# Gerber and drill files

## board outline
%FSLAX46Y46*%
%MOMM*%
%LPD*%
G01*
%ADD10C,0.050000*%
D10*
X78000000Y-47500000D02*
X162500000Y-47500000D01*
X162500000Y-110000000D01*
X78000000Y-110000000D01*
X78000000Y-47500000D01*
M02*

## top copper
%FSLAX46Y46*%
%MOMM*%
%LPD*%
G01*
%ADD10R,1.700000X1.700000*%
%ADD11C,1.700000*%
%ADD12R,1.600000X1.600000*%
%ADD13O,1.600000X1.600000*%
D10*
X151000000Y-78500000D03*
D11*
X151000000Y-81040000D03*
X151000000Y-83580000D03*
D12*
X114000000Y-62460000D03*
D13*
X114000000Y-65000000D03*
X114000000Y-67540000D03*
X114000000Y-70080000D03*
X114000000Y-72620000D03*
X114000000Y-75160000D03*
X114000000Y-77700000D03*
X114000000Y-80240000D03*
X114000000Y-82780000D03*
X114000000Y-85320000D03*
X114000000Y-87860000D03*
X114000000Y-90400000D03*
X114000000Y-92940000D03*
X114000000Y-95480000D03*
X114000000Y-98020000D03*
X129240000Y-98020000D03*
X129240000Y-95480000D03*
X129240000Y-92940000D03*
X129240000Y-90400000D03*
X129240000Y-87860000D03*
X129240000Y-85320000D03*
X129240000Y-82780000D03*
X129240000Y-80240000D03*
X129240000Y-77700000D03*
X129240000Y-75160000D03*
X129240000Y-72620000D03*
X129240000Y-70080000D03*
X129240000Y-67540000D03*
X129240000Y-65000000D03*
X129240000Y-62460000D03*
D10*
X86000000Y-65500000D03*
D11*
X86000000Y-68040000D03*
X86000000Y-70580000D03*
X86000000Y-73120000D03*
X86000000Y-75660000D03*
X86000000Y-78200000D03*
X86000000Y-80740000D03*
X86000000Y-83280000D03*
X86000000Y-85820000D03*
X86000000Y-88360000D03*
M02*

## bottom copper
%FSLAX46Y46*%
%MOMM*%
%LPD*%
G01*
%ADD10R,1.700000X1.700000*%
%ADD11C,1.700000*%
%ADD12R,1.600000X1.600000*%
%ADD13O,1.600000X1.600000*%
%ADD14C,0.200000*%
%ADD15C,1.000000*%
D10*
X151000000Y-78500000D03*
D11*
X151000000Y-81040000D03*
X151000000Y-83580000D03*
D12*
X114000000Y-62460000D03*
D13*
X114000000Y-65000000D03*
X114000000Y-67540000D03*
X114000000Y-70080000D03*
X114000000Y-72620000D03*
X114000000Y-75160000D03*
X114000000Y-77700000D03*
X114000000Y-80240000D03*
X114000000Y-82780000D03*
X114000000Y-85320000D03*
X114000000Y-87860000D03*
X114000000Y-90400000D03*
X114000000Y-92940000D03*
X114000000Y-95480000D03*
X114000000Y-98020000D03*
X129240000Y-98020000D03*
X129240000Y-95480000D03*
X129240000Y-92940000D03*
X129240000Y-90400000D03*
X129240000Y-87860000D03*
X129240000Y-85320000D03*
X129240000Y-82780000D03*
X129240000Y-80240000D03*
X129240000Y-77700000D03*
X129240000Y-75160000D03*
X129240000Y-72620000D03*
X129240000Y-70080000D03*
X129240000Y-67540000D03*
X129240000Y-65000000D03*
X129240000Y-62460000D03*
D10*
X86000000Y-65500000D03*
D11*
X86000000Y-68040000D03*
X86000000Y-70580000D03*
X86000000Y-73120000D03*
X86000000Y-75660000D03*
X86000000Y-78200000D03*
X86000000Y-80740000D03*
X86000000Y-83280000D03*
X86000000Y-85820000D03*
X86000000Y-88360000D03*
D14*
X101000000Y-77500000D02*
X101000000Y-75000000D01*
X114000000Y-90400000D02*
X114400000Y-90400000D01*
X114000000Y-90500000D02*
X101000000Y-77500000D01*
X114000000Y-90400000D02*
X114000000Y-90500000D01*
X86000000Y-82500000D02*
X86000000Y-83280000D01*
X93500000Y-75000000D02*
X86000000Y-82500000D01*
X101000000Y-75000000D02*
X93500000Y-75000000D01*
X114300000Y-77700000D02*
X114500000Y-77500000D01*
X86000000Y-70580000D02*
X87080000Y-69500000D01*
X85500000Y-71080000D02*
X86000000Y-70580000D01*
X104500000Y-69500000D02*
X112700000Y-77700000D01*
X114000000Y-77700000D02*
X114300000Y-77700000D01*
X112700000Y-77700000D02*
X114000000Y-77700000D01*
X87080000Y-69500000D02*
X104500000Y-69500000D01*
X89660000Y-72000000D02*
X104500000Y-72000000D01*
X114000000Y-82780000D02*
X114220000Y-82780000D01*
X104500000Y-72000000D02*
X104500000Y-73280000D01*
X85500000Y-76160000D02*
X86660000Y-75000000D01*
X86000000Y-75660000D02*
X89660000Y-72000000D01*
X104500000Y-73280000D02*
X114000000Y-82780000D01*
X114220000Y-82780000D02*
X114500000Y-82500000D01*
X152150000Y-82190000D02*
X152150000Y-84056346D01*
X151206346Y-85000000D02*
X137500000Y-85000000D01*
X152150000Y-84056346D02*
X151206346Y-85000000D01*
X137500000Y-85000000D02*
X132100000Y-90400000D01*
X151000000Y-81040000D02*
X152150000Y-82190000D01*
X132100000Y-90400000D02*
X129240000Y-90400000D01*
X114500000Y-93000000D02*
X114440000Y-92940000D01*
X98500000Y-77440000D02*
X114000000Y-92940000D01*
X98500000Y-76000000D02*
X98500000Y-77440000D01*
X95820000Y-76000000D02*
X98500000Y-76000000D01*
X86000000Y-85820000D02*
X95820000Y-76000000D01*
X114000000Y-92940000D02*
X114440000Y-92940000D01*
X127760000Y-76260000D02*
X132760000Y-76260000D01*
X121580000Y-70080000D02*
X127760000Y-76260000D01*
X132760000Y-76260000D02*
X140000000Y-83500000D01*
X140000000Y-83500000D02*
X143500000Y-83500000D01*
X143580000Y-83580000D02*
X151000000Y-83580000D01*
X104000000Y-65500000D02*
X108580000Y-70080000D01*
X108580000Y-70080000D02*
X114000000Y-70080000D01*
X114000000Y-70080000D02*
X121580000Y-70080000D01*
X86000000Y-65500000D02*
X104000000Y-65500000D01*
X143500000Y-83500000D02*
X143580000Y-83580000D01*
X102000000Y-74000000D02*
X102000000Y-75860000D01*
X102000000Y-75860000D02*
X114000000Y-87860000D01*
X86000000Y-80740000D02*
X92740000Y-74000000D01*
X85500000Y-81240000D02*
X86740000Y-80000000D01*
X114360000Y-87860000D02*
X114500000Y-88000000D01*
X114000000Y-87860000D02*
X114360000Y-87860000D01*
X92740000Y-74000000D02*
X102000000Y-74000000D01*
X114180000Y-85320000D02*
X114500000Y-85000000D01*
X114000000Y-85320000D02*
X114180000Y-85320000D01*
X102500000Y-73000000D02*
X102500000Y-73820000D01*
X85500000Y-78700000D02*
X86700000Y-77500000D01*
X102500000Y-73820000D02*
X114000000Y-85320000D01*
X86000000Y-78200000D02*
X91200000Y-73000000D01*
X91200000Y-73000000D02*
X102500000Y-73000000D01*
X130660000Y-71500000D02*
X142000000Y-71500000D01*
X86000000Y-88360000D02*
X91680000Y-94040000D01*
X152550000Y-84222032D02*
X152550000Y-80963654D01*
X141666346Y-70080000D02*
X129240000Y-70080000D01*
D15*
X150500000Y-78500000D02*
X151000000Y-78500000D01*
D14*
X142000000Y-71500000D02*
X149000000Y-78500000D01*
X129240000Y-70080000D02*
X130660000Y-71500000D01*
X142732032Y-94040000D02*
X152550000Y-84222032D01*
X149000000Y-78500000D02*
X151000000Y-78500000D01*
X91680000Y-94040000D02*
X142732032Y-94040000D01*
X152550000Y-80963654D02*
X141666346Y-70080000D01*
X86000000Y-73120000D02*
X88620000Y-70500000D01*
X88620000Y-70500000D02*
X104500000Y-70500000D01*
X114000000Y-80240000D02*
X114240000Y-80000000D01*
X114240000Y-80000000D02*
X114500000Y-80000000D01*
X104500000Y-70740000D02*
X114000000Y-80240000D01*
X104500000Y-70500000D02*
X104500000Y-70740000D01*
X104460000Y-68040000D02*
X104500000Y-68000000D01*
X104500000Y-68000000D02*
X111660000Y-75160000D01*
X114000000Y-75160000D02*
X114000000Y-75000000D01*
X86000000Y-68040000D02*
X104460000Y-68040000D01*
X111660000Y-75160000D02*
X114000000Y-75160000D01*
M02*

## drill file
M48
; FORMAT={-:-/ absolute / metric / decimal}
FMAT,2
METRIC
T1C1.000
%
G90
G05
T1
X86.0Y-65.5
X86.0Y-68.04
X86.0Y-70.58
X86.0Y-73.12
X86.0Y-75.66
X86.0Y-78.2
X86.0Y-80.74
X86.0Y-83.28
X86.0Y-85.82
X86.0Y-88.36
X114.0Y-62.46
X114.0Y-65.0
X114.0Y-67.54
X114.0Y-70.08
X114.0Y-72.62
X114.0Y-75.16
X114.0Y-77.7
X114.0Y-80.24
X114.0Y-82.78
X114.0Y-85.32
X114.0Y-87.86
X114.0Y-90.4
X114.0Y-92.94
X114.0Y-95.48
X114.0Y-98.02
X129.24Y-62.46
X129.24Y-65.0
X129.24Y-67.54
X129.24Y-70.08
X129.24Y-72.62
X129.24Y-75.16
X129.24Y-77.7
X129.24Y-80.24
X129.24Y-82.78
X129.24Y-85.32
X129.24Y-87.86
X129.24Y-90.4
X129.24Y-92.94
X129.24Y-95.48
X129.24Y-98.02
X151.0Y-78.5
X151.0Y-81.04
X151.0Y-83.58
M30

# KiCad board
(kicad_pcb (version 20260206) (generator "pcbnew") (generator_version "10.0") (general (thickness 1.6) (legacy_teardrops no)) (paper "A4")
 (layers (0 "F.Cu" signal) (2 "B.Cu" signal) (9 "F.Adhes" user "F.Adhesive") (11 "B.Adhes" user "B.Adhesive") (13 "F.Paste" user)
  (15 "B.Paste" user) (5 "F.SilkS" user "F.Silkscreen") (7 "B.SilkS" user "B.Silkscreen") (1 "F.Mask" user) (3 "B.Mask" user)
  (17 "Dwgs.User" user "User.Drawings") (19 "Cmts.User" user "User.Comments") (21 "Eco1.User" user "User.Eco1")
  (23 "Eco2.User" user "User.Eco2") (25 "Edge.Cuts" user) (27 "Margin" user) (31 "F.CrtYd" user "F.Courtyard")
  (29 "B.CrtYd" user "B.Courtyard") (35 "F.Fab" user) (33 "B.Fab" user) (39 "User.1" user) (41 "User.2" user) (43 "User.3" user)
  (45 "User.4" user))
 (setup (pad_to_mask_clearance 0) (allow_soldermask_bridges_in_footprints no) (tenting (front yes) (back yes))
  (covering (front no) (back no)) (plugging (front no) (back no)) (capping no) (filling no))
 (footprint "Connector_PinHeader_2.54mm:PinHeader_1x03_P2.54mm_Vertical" (layer "F.Cu") (at 151 78.5)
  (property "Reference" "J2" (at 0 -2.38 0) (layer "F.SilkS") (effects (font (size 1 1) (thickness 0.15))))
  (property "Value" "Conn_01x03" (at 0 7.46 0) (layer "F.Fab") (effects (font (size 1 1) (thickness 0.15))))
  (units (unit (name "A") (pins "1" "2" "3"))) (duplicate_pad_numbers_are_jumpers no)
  (pad "1" thru_hole rect (at 0 0) (size 1.7 1.7) (drill 1) (layers "*.Cu" "*.Mask") (remove_unused_layers no) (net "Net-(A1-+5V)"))
  (pad "2" thru_hole circle (at 0 2.54) (size 1.7 1.7) (drill 1) (layers "*.Cu" "*.Mask") (remove_unused_layers no) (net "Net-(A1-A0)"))
  (pad "3" thru_hole circle (at 0 5.08) (size 1.7 1.7) (drill 1) (layers "*.Cu" "*.Mask") (remove_unused_layers no) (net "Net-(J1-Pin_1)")))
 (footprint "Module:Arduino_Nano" (layer "F.Cu") (at 114 62.46)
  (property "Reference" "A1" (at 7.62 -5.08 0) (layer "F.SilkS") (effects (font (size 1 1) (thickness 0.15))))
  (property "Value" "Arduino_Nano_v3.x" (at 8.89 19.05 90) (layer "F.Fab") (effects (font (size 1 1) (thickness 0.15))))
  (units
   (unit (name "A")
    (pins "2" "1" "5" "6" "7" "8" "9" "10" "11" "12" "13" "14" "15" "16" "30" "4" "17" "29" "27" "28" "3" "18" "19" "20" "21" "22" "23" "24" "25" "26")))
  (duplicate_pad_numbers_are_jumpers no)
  (pad "1" thru_hole rect (at 0 0) (size 1.6 1.6) (drill 1) (layers "*.Cu" "*.Mask") (remove_unused_layers no)
   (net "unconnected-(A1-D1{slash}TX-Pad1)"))
  (pad "2" thru_hole oval (at 0 2.54) (size 1.6 1.6) (drill 1) (layers "*.Cu" "*.Mask") (remove_unused_layers no)
   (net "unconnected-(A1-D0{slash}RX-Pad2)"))
  (pad "3" thru_hole oval (at 0 5.08) (size 1.6 1.6) (drill 1) (layers "*.Cu" "*.Mask") (remove_unused_layers no)
   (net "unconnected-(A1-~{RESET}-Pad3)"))
  (pad "4" thru_hole oval (at 0 7.62) (size 1.6 1.6) (drill 1) (layers "*.Cu" "*.Mask") (remove_unused_layers no) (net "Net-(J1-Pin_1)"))
  (pad "5" thru_hole oval (at 0 10.16) (size 1.6 1.6) (drill 1) (layers "*.Cu" "*.Mask") (remove_unused_layers no)
   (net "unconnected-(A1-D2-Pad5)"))
  (pad "6" thru_hole oval (at 0 12.7) (size 1.6 1.6) (drill 1) (layers "*.Cu" "*.Mask") (remove_unused_layers no) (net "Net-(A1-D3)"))
  (pad "7" thru_hole oval (at 0 15.24) (size 1.6 1.6) (drill 1) (layers "*.Cu" "*.Mask") (remove_unused_layers no) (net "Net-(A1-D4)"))
  (pad "8" thru_hole oval (at 0 17.78) (size 1.6 1.6) (drill 1) (layers "*.Cu" "*.Mask") (remove_unused_layers no) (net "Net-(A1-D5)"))
  (pad "9" thru_hole oval (at 0 20.32) (size 1.6 1.6) (drill 1) (layers "*.Cu" "*.Mask") (remove_unused_layers no) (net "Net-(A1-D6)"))
  (pad "10" thru_hole oval (at 0 22.86) (size 1.6 1.6) (drill 1) (layers "*.Cu" "*.Mask") (remove_unused_layers no) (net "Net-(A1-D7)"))
  (pad "11" thru_hole oval (at 0 25.4) (size 1.6 1.6) (drill 1) (layers "*.Cu" "*.Mask") (remove_unused_layers no) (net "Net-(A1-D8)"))
  (pad "12" thru_hole oval (at 0 27.94) (size 1.6 1.6) (drill 1) (layers "*.Cu" "*.Mask") (remove_unused_layers no) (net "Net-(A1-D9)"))
  (pad "13" thru_hole oval (at 0 30.48) (size 1.6 1.6) (drill 1) (layers "*.Cu" "*.Mask") (remove_unused_layers no) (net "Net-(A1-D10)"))
  (pad "14" thru_hole oval (at 0 33.02) (size 1.6 1.6) (drill 1) (layers "*.Cu" "*.Mask") (remove_unused_layers no)
   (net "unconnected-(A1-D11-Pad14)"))
  (pad "15" thru_hole oval (at 0 35.56) (size 1.6 1.6) (drill 1) (layers "*.Cu" "*.Mask") (remove_unused_layers no)
   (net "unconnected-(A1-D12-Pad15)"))
  (pad "16" thru_hole oval (at 15.24 35.56) (size 1.6 1.6) (drill 1) (layers "*.Cu" "*.Mask") (remove_unused_layers no)
   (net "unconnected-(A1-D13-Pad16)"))
  (pad "17" thru_hole oval (at 15.24 33.02) (size 1.6 1.6) (drill 1) (layers "*.Cu" "*.Mask") (remove_unused_layers no)
   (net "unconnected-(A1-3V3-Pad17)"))
  (pad "18" thru_hole oval (at 15.24 30.48) (size 1.6 1.6) (drill 1) (layers "*.Cu" "*.Mask") (remove_unused_layers no)
   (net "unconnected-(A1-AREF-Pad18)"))
  (pad "19" thru_hole oval (at 15.24 27.94) (size 1.6 1.6) (drill 1) (layers "*.Cu" "*.Mask") (remove_unused_layers no) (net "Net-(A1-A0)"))
  (pad "20" thru_hole oval (at 15.24 25.4) (size 1.6 1.6) (drill 1) (layers "*.Cu" "*.Mask") (remove_unused_layers no)
   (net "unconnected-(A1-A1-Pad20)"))
  (pad "21" thru_hole oval (at 15.24 22.86) (size 1.6 1.6) (drill 1) (layers "*.Cu" "*.Mask") (remove_unused_layers no)
   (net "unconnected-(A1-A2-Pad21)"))
  (pad "22" thru_hole oval (at 15.24 20.32) (size 1.6 1.6) (drill 1) (layers "*.Cu" "*.Mask") (remove_unused_layers no)
   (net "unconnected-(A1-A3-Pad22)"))
  (pad "23" thru_hole oval (at 15.24 17.78) (size 1.6 1.6) (drill 1) (layers "*.Cu" "*.Mask") (remove_unused_layers no)
   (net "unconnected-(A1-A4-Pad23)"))
  (pad "24" thru_hole oval (at 15.24 15.24) (size 1.6 1.6) (drill 1) (layers "*.Cu" "*.Mask") (remove_unused_layers no)
   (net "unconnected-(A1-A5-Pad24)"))
  (pad "25" thru_hole oval (at 15.24 12.7) (size 1.6 1.6) (drill 1) (layers "*.Cu" "*.Mask") (remove_unused_layers no)
   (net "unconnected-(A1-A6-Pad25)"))
  (pad "26" thru_hole oval (at 15.24 10.16) (size 1.6 1.6) (drill 1) (layers "*.Cu" "*.Mask") (remove_unused_layers no)
   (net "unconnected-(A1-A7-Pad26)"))
  (pad "27" thru_hole oval (at 15.24 7.62) (size 1.6 1.6) (drill 1) (layers "*.Cu" "*.Mask") (remove_unused_layers no) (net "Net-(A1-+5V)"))
  (pad "28" thru_hole oval (at 15.24 5.08) (size 1.6 1.6) (drill 1) (layers "*.Cu" "*.Mask") (remove_unused_layers no)
   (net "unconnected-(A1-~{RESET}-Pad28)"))
  (pad "29" thru_hole oval (at 15.24 2.54) (size 1.6 1.6) (drill 1) (layers "*.Cu" "*.Mask") (remove_unused_layers no)
   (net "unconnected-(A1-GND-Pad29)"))
  (pad "30" thru_hole oval (at 15.24 0) (size 1.6 1.6) (drill 1) (layers "*.Cu" "*.Mask") (remove_unused_layers no)
   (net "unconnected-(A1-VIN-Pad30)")))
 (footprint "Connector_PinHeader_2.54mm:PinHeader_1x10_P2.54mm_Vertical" (layer "F.Cu") (at 86 65.5)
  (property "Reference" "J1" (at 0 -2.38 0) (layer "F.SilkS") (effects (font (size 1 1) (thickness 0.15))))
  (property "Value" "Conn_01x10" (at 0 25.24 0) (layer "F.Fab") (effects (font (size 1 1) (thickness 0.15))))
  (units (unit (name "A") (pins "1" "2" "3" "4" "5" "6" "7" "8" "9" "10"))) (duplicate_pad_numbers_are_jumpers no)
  (pad "1" thru_hole rect (at 0 0) (size 1.7 1.7) (drill 1) (layers "*.Cu" "*.Mask") (remove_unused_layers no) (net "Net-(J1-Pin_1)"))
  (pad "2" thru_hole circle (at 0 2.54) (size 1.7 1.7) (drill 1) (layers "*.Cu" "*.Mask") (remove_unused_layers no) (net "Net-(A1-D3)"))
  (pad "3" thru_hole circle (at 0 5.08) (size 1.7 1.7) (drill 1) (layers "*.Cu" "*.Mask") (remove_unused_layers no) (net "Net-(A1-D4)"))
  (pad "4" thru_hole circle (at 0 7.62) (size 1.7 1.7) (drill 1) (layers "*.Cu" "*.Mask") (remove_unused_layers no) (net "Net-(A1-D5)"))
  (pad "5" thru_hole circle (at 0 10.16) (size 1.7 1.7) (drill 1) (layers "*.Cu" "*.Mask") (remove_unused_layers no) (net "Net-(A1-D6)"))
  (pad "6" thru_hole circle (at 0 12.7) (size 1.7 1.7) (drill 1) (layers "*.Cu" "*.Mask") (remove_unused_layers no) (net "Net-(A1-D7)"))
  (pad "7" thru_hole circle (at 0 15.24) (size 1.7 1.7) (drill 1) (layers "*.Cu" "*.Mask") (remove_unused_layers no) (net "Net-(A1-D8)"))
  (pad "8" thru_hole circle (at 0 17.78) (size 1.7 1.7) (drill 1) (layers "*.Cu" "*.Mask") (remove_unused_layers no) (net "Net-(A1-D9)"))
  (pad "9" thru_hole circle (at 0 20.32) (size 1.7 1.7) (drill 1) (layers "*.Cu" "*.Mask") (remove_unused_layers no) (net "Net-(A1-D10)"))
  (pad "10" thru_hole circle (at 0 22.86) (size 1.7 1.7) (drill 1) (layers "*.Cu" "*.Mask") (remove_unused_layers no) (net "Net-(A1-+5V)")))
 (gr_rect (start 78 47.5) (end 162.5 110) (stroke (width 0.05) (type default)) (fill no) (layer "Edge.Cuts"))
 (segment (start 101 77.5) (end 101 75) (width 0.2) (layer "B.Cu") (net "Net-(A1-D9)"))
 (segment (start 114 90.4) (end 114.4 90.4) (width 0.2) (layer "B.Cu") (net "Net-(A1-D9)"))
 (segment (start 114 90.5) (end 101 77.5) (width 0.2) (layer "B.Cu") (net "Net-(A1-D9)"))
 (segment (start 114 90.4) (end 114 90.5) (width 0.2) (layer "B.Cu") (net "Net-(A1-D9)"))
 (segment (start 86 82.5) (end 86 83.28) (width 0.2) (layer "B.Cu") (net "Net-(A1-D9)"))
 (segment (start 93.5 75) (end 86 82.5) (width 0.2) (layer "B.Cu") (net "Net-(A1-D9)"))
 (segment (start 101 75) (end 93.5 75) (width 0.2) (layer "B.Cu") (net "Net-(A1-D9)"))
 (segment (start 114.3 77.7) (end 114.5 77.5) (width 0.2) (layer "B.Cu") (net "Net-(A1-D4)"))
 (segment (start 86 70.58) (end 87.08 69.5) (width 0.2) (layer "B.Cu") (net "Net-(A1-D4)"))
 (segment (start 85.5 71.08) (end 86 70.58) (width 0.2) (layer "B.Cu") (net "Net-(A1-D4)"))
 (segment (start 104.5 69.5) (end 112.7 77.7) (width 0.2) (layer "B.Cu") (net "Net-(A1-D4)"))
 (segment (start 114 77.7) (end 114.3 77.7) (width 0.2) (layer "B.Cu") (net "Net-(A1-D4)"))
 (segment (start 112.7 77.7) (end 114 77.7) (width 0.2) (layer "B.Cu") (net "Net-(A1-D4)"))
 (segment (start 87.08 69.5) (end 104.5 69.5) (width 0.2) (layer "B.Cu") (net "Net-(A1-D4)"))
 (segment (start 89.66 72) (end 104.5 72) (width 0.2) (layer "B.Cu") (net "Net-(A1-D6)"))
 (segment (start 114 82.78) (end 114.22 82.78) (width 0.2) (layer "B.Cu") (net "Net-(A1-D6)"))
 (segment (start 104.5 72) (end 104.5 73.28) (width 0.2) (layer "B.Cu") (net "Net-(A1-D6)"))
 (segment (start 85.5 76.16) (end 86.66 75) (width 0.2) (layer "B.Cu") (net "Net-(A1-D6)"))
 (segment (start 86 75.66) (end 89.66 72) (width 0.2) (layer "B.Cu") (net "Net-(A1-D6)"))
 (segment (start 104.5 73.28) (end 114 82.78) (width 0.2) (layer "B.Cu") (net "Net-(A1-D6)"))
 (segment (start 114.22 82.78) (end 114.5 82.5) (width 0.2) (layer "B.Cu") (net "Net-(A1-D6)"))
 (segment (start 152.15 82.19) (end 152.15 84.056346) (width 0.2) (layer "B.Cu") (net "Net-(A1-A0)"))
 (segment (start 151.206346 85) (end 137.5 85) (width 0.2) (layer "B.Cu") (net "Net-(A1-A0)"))
 (segment (start 152.15 84.056346) (end 151.206346 85) (width 0.2) (layer "B.Cu") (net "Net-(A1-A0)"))
 (segment (start 137.5 85) (end 132.1 90.4) (width 0.2) (layer "B.Cu") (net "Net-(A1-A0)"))
 (segment (start 151 81.04) (end 152.15 82.19) (width 0.2) (layer "B.Cu") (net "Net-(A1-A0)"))
 (segment (start 132.1 90.4) (end 129.24 90.4) (width 0.2) (layer "B.Cu") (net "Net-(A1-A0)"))
 (segment (start 114.5 93) (end 114.44 92.94) (width 0.2) (layer "B.Cu") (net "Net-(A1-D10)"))
 (segment (start 98.5 77.44) (end 114 92.94) (width 0.2) (layer "B.Cu") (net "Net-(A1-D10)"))
 (segment (start 98.5 76) (end 98.5 77.44) (width 0.2) (layer "B.Cu") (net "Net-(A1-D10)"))
 (segment (start 95.82 76) (end 98.5 76) (width 0.2) (layer "B.Cu") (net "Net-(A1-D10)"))
 (segment (start 86 85.82) (end 95.82 76) (width 0.2) (layer "B.Cu") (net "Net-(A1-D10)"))
 (segment (start 114 92.94) (end 114.44 92.94) (width 0.2) (layer "B.Cu") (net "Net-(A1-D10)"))
 (segment (start 127.76 76.26) (end 132.76 76.26) (width 0.2) (layer "B.Cu") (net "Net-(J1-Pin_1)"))
 (segment (start 121.58 70.08) (end 127.76 76.26) (width 0.2) (layer "B.Cu") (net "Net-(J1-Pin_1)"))
 (segment (start 132.76 76.26) (end 140 83.5) (width 0.2) (layer "B.Cu") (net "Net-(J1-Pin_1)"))
 (segment (start 140 83.5) (end 143.5 83.5) (width 0.2) (layer "B.Cu") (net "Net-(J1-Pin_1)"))
 (segment (start 143.58 83.58) (end 151 83.58) (width 0.2) (layer "B.Cu") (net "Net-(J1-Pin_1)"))
 (segment (start 104 65.5) (end 108.58 70.08) (width 0.2) (layer "B.Cu") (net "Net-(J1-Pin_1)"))
 (segment (start 108.58 70.08) (end 114 70.08) (width 0.2) (layer "B.Cu") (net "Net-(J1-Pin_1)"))
 (segment (start 114 70.08) (end 121.58 70.08) (width 0.2) (layer "B.Cu") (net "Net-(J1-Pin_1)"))
 (segment (start 86 65.5) (end 104 65.5) (width 0.2) (layer "B.Cu") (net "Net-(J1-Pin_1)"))
 (segment (start 143.5 83.5) (end 143.58 83.58) (width 0.2) (layer "B.Cu") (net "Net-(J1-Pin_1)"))
 (segment (start 102 74) (end 102 75.86) (width 0.2) (layer "B.Cu") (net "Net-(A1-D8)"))
 (segment (start 102 75.86) (end 114 87.86) (width 0.2) (layer "B.Cu") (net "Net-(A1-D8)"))
 (segment (start 86 80.74) (end 92.74 74) (width 0.2) (layer "B.Cu") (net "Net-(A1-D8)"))
 (segment (start 85.5 81.24) (end 86.74 80) (width 0.2) (layer "B.Cu") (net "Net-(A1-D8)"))
 (segment (start 114.36 87.86) (end 114.5 88) (width 0.2) (layer "B.Cu") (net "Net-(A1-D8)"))
 (segment (start 114 87.86) (end 114.36 87.86) (width 0.2) (layer "B.Cu") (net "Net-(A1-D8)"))
 (segment (start 92.74 74) (end 102 74) (width 0.2) (layer "B.Cu") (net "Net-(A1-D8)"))
 (segment (start 114.18 85.32) (end 114.5 85) (width 0.2) (layer "B.Cu") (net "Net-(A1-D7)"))
 (segment (start 114 85.32) (end 114.18 85.32) (width 0.2) (layer "B.Cu") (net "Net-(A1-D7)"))
 (segment (start 102.5 73) (end 102.5 73.82) (width 0.2) (layer "B.Cu") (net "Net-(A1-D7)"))
 (segment (start 85.5 78.7) (end 86.7 77.5) (width 0.2) (layer "B.Cu") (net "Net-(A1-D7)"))
 (segment (start 102.5 73.82) (end 114 85.32) (width 0.2) (layer "B.Cu") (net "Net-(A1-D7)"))
 (segment (start 86 78.2) (end 91.2 73) (width 0.2) (layer "B.Cu") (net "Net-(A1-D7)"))
 (segment (start 91.2 73) (end 102.5 73) (width 0.2) (layer "B.Cu") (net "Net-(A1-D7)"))
 (segment (start 130.66 71.5) (end 142 71.5) (width 0.2) (layer "B.Cu") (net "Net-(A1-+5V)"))
 (segment (start 86 88.36) (end 91.68 94.04) (width 0.2) (layer "B.Cu") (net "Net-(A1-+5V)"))
 (segment (start 152.55 84.222032) (end 152.55 80.963654) (width 0.2) (layer "B.Cu") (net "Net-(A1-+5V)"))
 (segment (start 141.666346 70.08) (end 129.24 70.08) (width 0.2) (layer "B.Cu") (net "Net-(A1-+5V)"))
 (segment (start 150.5 78.5) (end 151 78.5) (width 1) (layer "B.Cu") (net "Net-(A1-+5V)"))
 (segment (start 142 71.5) (end 149 78.5) (width 0.2) (layer "B.Cu") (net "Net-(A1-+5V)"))
 (segment (start 129.24 70.08) (end 130.66 71.5) (width 0.2) (layer "B.Cu") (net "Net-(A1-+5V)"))
 (segment (start 142.732032 94.04) (end 152.55 84.222032) (width 0.2) (layer "B.Cu") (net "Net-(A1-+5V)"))
 (segment (start 149 78.5) (end 151 78.5) (width 0.2) (layer "B.Cu") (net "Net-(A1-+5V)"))
 (segment (start 91.68 94.04) (end 142.732032 94.04) (width 0.2) (layer "B.Cu") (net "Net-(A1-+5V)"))
 (segment (start 152.55 80.963654) (end 141.666346 70.08) (width 0.2) (layer "B.Cu") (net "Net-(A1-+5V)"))
 (segment (start 86 73.12) (end 88.62 70.5) (width 0.2) (layer "B.Cu") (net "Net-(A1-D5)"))
 (segment (start 88.62 70.5) (end 104.5 70.5) (width 0.2) (layer "B.Cu") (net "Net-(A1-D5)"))
 (segment (start 114 80.24) (end 114.24 80) (width 0.2) (layer "B.Cu") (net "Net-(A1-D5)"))
 (segment (start 114.24 80) (end 114.5 80) (width 0.2) (layer "B.Cu") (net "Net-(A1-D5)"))
 (segment (start 104.5 70.74) (end 114 80.24) (width 0.2) (layer "B.Cu") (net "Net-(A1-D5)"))
 (segment (start 104.5 70.5) (end 104.5 70.74) (width 0.2) (layer "B.Cu") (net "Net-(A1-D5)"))
 (segment (start 104.46 68.04) (end 104.5 68) (width 0.2) (layer "B.Cu") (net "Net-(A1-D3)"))
 (segment (start 104.5 68) (end 111.66 75.16) (width 0.2) (layer "B.Cu") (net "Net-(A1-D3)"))
 (segment (start 114 75.16) (end 114 75) (width 0.2) (layer "B.Cu") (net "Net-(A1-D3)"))
 (segment (start 86 68.04) (end 104.46 68.04) (width 0.2) (layer "B.Cu") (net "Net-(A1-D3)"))
 (segment (start 111.66 75.16) (end 114 75.16) (width 0.2) (layer "B.Cu") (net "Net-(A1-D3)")))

